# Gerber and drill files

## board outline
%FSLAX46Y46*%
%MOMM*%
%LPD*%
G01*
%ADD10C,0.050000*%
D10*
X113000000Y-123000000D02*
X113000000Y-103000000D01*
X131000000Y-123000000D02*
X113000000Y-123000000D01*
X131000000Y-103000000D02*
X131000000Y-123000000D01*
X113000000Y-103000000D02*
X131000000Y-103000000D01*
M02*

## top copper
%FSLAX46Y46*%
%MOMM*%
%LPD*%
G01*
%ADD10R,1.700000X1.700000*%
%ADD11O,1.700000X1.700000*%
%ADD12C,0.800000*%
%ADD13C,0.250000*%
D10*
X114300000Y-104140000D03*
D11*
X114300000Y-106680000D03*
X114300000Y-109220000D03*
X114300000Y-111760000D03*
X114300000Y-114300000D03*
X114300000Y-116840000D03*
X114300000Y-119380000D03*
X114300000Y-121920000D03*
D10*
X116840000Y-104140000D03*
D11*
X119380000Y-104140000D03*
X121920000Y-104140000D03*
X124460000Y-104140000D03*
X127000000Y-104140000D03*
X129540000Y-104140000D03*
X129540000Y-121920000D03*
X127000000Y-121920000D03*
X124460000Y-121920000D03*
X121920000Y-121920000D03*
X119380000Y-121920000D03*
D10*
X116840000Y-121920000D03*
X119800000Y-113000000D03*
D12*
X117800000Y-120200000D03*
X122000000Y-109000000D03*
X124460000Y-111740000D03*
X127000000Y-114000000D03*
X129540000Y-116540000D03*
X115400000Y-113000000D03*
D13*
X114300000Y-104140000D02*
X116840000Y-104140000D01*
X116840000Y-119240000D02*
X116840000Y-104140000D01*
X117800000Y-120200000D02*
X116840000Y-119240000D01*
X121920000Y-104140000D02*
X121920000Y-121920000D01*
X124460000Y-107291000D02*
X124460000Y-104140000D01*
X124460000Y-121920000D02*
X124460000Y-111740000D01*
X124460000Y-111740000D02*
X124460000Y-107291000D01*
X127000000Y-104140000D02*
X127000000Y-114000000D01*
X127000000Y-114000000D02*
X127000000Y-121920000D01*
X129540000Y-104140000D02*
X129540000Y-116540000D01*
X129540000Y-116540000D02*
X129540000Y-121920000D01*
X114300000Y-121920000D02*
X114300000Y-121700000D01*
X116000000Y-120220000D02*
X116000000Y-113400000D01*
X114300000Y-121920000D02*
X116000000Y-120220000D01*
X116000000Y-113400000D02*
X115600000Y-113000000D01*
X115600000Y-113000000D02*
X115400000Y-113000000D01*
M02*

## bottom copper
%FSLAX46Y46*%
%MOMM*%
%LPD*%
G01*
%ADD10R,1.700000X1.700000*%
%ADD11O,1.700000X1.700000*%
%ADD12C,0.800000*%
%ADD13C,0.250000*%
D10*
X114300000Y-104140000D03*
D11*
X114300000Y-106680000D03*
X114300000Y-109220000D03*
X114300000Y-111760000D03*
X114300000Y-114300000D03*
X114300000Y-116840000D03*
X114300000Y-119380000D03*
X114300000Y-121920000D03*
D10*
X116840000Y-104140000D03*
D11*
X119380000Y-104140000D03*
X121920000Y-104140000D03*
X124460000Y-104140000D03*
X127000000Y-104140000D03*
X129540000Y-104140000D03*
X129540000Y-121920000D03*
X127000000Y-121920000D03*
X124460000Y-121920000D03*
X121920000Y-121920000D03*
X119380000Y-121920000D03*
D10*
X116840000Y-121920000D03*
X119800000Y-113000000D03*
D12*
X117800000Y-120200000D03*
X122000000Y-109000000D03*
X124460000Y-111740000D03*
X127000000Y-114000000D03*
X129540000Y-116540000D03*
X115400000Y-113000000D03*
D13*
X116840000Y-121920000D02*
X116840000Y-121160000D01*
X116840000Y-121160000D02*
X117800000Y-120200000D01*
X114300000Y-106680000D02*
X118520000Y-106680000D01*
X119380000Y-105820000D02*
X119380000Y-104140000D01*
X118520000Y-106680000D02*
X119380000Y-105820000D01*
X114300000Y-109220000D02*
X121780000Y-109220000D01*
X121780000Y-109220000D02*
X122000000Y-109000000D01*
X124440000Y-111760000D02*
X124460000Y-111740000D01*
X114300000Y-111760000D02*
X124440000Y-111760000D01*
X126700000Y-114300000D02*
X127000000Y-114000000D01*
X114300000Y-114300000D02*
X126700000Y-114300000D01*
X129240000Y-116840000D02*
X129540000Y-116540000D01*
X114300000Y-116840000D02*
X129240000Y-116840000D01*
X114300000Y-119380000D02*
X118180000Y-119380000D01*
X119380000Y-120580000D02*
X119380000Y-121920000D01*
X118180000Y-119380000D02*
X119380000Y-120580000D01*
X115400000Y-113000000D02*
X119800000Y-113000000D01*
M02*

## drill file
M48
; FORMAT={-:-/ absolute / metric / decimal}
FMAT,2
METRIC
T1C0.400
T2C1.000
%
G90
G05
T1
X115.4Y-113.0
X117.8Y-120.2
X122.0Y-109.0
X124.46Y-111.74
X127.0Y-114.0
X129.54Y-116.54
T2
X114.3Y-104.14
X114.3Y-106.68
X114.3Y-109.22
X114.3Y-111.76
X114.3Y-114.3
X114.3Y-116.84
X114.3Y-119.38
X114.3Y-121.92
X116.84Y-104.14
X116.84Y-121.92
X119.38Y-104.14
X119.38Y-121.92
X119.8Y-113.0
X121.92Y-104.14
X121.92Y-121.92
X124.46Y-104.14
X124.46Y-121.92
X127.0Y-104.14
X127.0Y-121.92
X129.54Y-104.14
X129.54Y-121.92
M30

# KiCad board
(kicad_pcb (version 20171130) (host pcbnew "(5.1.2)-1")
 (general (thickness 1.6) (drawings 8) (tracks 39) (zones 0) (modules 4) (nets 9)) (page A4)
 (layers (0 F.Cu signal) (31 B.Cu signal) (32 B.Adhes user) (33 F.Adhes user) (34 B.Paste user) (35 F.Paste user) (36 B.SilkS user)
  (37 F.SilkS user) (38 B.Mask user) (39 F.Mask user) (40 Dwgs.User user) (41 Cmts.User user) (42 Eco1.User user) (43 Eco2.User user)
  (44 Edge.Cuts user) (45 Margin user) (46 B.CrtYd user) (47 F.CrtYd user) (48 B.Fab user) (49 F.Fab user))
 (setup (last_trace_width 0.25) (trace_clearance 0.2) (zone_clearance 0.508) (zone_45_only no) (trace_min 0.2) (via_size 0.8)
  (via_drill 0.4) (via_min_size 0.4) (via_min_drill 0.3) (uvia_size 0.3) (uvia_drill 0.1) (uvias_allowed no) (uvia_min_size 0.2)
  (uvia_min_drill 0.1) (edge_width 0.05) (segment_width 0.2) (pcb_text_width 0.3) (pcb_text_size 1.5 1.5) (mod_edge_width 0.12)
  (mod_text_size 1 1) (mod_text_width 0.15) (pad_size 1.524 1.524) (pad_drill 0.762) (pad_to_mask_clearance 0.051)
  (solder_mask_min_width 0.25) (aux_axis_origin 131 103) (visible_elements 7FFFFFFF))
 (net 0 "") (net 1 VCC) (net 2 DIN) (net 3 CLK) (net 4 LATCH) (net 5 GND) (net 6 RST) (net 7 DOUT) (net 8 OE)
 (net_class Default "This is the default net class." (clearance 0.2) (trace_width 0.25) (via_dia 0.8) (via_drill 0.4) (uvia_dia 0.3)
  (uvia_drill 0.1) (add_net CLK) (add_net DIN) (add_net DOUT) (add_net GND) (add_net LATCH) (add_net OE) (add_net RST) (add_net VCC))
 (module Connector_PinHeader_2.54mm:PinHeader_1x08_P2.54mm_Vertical (layer F.Cu) (at 114.3 104.14)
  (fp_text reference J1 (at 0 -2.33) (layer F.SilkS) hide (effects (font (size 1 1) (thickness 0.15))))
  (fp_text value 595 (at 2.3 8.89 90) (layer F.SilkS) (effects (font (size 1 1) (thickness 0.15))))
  (pad 1 thru_hole rect (at 0 0) (size 1.7 1.7) (drill 1) (layers *.Cu *.Mask) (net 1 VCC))
  (pad 2 thru_hole oval (at 0 2.54) (size 1.7 1.7) (drill 1) (layers *.Cu *.Mask) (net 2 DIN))
  (pad 3 thru_hole oval (at 0 5.08) (size 1.7 1.7) (drill 1) (layers *.Cu *.Mask) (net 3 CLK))
  (pad 4 thru_hole oval (at 0 7.62) (size 1.7 1.7) (drill 1) (layers *.Cu *.Mask) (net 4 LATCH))
  (pad 5 thru_hole oval (at 0 10.16) (size 1.7 1.7) (drill 1) (layers *.Cu *.Mask) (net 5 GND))
  (pad 6 thru_hole oval (at 0 12.7) (size 1.7 1.7) (drill 1) (layers *.Cu *.Mask) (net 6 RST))
  (pad 7 thru_hole oval (at 0 15.24) (size 1.7 1.7) (drill 1) (layers *.Cu *.Mask) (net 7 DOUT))
  (pad 8 thru_hole oval (at 0 17.78) (size 1.7 1.7) (drill 1) (layers *.Cu *.Mask) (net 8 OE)))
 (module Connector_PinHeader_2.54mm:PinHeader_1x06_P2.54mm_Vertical (layer F.Cu) (at 116.84 104.14 90)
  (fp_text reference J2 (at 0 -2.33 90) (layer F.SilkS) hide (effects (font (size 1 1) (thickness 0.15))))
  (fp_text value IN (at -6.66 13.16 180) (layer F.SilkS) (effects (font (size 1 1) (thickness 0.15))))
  (pad 1 thru_hole rect (at 0 0 90) (size 1.7 1.7) (drill 1) (layers *.Cu *.Mask) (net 1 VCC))
  (pad 2 thru_hole oval (at 0 2.54 90) (size 1.7 1.7) (drill 1) (layers *.Cu *.Mask) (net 2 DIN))
  (pad 3 thru_hole oval (at 0 5.08 90) (size 1.7 1.7) (drill 1) (layers *.Cu *.Mask) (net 3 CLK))
  (pad 4 thru_hole oval (at 0 7.62 90) (size 1.7 1.7) (drill 1) (layers *.Cu *.Mask) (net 4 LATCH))
  (pad 5 thru_hole oval (at 0 10.16 90) (size 1.7 1.7) (drill 1) (layers *.Cu *.Mask) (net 5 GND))
  (pad 6 thru_hole oval (at 0 12.7 90) (size 1.7 1.7) (drill 1) (layers *.Cu *.Mask) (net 6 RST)))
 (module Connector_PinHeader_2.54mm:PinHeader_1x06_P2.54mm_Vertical (layer F.Cu) (at 116.84 121.92 90)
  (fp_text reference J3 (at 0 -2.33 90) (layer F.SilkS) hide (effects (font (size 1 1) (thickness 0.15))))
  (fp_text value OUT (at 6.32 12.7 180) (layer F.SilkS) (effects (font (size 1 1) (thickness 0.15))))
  (pad 6 thru_hole oval (at 0 12.7 90) (size 1.7 1.7) (drill 1) (layers *.Cu *.Mask) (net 6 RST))
  (pad 5 thru_hole oval (at 0 10.16 90) (size 1.7 1.7) (drill 1) (layers *.Cu *.Mask) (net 5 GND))
  (pad 4 thru_hole oval (at 0 7.62 90) (size 1.7 1.7) (drill 1) (layers *.Cu *.Mask) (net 4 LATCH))
  (pad 3 thru_hole oval (at 0 5.08 90) (size 1.7 1.7) (drill 1) (layers *.Cu *.Mask) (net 3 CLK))
  (pad 2 thru_hole oval (at 0 2.54 90) (size 1.7 1.7) (drill 1) (layers *.Cu *.Mask) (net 7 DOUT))
  (pad 1 thru_hole rect (at 0 0 90) (size 1.7 1.7) (drill 1) (layers *.Cu *.Mask) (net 1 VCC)))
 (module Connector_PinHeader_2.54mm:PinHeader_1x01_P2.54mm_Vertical (layer F.Cu) (at 119.8 113)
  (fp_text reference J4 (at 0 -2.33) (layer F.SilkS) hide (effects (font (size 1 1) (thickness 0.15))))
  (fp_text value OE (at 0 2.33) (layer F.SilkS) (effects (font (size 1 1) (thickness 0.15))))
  (pad 1 thru_hole rect (at 0 0) (size 1.7 1.7) (drill 1) (layers *.Cu *.Mask) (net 8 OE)))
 (gr_line (start 113 123) (end 113 103) (layer Edge.Cuts) (width 0.05))
 (gr_line (start 131 123) (end 113 123) (layer Edge.Cuts) (width 0.05))
 (gr_line (start 131 103) (end 131 123) (layer Edge.Cuts) (width 0.05))
 (gr_line (start 113 103) (end 131 103) (layer Edge.Cuts) (width 0.05))
 (segment (start 114.3 104.14) (end 116.84 104.14) (width 0.25) (layer F.Cu) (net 1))
 (via (at 117.8 120.2) (size 0.8) (drill 0.4) (layers F.Cu B.Cu) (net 1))
 (segment (start 116.84 121.92) (end 116.84 121.16) (width 0.25) (layer B.Cu) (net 1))
 (segment (start 116.84 121.16) (end 117.8 120.2) (width 0.25) (layer B.Cu) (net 1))
 (segment (start 116.84 119.24) (end 116.84 104.14) (width 0.25) (layer F.Cu) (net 1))
 (segment (start 117.8 120.2) (end 116.84 119.24) (width 0.25) (layer F.Cu) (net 1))
 (segment (start 114.3 106.68) (end 118.52 106.68) (width 0.25) (layer B.Cu) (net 2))
 (segment (start 119.38 105.82) (end 119.38 104.14) (width 0.25) (layer B.Cu) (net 2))
 (segment (start 118.52 106.68) (end 119.38 105.82) (width 0.25) (layer B.Cu) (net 2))
 (segment (start 121.92 104.14) (end 121.92 121.92) (width 0.25) (layer F.Cu) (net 3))
 (via (at 122 109) (size 0.8) (drill 0.4) (layers F.Cu B.Cu) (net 3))
 (segment (start 114.3 109.22) (end 121.78 109.22) (width 0.25) (layer B.Cu) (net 3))
 (segment (start 121.78 109.22) (end 122 109) (width 0.25) (layer B.Cu) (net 3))
 (segment (start 124.46 107.291) (end 124.46 104.14) (width 0.25) (layer F.Cu) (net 4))
 (via (at 124.46 111.74) (size 0.8) (drill 0.4) (layers F.Cu B.Cu) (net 4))
 (segment (start 124.44 111.76) (end 124.46 111.74) (width 0.25) (layer B.Cu) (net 4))
 (segment (start 114.3 111.76) (end 124.44 111.76) (width 0.25) (layer B.Cu) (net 4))
 (segment (start 124.46 121.92) (end 124.46 111.74) (width 0.25) (layer F.Cu) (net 4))
 (segment (start 124.46 111.74) (end 124.46 107.291) (width 0.25) (layer F.Cu) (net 4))
 (via (at 127 114) (size 0.8) (drill 0.4) (layers F.Cu B.Cu) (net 5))
 (segment (start 126.7 114.3) (end 127 114) (width 0.25) (layer B.Cu) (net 5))
 (segment (start 114.3 114.3) (end 126.7 114.3) (width 0.25) (layer B.Cu) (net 5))
 (segment (start 127 104.14) (end 127 114) (width 0.25) (layer F.Cu) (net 5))
 (segment (start 127 114) (end 127 121.92) (width 0.25) (layer F.Cu) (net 5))
 (via (at 129.54 116.54) (size 0.8) (drill 0.4) (layers F.Cu B.Cu) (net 6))
 (segment (start 129.24 116.84) (end 129.54 116.54) (width 0.25) (layer B.Cu) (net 6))
 (segment (start 114.3 116.84) (end 129.24 116.84) (width 0.25) (layer B.Cu) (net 6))
 (segment (start 129.54 104.14) (end 129.54 116.54) (width 0.25) (layer F.Cu) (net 6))
 (segment (start 129.54 116.54) (end 129.54 121.92) (width 0.25) (layer F.Cu) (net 6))
 (segment (start 114.3 119.38) (end 118.18 119.38) (width 0.25) (layer B.Cu) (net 7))
 (segment (start 119.38 120.58) (end 119.38 121.92) (width 0.25) (layer B.Cu) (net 7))
 (segment (start 118.18 119.38) (end 119.38 120.58) (width 0.25) (layer B.Cu) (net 7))
 (segment (start 114.3 121.92) (end 114.3 121.7) (width 0.25) (layer F.Cu) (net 8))
 (segment (start 116 120.22) (end 116 113.4) (width 0.25) (layer F.Cu) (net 8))
 (segment (start 114.3 121.92) (end 116 120.22) (width 0.25) (layer F.Cu) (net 8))
 (via (at 115.4 113) (size 0.8) (drill 0.4) (layers F.Cu B.Cu) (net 8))
 (segment (start 116 113.4) (end 115.6 113) (width 0.25) (layer F.Cu) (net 8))
 (segment (start 115.6 113) (end 115.4 113) (width 0.25) (layer F.Cu) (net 8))
 (segment (start 115.4 113) (end 119.8 113) (width 0.25) (layer B.Cu) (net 8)))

